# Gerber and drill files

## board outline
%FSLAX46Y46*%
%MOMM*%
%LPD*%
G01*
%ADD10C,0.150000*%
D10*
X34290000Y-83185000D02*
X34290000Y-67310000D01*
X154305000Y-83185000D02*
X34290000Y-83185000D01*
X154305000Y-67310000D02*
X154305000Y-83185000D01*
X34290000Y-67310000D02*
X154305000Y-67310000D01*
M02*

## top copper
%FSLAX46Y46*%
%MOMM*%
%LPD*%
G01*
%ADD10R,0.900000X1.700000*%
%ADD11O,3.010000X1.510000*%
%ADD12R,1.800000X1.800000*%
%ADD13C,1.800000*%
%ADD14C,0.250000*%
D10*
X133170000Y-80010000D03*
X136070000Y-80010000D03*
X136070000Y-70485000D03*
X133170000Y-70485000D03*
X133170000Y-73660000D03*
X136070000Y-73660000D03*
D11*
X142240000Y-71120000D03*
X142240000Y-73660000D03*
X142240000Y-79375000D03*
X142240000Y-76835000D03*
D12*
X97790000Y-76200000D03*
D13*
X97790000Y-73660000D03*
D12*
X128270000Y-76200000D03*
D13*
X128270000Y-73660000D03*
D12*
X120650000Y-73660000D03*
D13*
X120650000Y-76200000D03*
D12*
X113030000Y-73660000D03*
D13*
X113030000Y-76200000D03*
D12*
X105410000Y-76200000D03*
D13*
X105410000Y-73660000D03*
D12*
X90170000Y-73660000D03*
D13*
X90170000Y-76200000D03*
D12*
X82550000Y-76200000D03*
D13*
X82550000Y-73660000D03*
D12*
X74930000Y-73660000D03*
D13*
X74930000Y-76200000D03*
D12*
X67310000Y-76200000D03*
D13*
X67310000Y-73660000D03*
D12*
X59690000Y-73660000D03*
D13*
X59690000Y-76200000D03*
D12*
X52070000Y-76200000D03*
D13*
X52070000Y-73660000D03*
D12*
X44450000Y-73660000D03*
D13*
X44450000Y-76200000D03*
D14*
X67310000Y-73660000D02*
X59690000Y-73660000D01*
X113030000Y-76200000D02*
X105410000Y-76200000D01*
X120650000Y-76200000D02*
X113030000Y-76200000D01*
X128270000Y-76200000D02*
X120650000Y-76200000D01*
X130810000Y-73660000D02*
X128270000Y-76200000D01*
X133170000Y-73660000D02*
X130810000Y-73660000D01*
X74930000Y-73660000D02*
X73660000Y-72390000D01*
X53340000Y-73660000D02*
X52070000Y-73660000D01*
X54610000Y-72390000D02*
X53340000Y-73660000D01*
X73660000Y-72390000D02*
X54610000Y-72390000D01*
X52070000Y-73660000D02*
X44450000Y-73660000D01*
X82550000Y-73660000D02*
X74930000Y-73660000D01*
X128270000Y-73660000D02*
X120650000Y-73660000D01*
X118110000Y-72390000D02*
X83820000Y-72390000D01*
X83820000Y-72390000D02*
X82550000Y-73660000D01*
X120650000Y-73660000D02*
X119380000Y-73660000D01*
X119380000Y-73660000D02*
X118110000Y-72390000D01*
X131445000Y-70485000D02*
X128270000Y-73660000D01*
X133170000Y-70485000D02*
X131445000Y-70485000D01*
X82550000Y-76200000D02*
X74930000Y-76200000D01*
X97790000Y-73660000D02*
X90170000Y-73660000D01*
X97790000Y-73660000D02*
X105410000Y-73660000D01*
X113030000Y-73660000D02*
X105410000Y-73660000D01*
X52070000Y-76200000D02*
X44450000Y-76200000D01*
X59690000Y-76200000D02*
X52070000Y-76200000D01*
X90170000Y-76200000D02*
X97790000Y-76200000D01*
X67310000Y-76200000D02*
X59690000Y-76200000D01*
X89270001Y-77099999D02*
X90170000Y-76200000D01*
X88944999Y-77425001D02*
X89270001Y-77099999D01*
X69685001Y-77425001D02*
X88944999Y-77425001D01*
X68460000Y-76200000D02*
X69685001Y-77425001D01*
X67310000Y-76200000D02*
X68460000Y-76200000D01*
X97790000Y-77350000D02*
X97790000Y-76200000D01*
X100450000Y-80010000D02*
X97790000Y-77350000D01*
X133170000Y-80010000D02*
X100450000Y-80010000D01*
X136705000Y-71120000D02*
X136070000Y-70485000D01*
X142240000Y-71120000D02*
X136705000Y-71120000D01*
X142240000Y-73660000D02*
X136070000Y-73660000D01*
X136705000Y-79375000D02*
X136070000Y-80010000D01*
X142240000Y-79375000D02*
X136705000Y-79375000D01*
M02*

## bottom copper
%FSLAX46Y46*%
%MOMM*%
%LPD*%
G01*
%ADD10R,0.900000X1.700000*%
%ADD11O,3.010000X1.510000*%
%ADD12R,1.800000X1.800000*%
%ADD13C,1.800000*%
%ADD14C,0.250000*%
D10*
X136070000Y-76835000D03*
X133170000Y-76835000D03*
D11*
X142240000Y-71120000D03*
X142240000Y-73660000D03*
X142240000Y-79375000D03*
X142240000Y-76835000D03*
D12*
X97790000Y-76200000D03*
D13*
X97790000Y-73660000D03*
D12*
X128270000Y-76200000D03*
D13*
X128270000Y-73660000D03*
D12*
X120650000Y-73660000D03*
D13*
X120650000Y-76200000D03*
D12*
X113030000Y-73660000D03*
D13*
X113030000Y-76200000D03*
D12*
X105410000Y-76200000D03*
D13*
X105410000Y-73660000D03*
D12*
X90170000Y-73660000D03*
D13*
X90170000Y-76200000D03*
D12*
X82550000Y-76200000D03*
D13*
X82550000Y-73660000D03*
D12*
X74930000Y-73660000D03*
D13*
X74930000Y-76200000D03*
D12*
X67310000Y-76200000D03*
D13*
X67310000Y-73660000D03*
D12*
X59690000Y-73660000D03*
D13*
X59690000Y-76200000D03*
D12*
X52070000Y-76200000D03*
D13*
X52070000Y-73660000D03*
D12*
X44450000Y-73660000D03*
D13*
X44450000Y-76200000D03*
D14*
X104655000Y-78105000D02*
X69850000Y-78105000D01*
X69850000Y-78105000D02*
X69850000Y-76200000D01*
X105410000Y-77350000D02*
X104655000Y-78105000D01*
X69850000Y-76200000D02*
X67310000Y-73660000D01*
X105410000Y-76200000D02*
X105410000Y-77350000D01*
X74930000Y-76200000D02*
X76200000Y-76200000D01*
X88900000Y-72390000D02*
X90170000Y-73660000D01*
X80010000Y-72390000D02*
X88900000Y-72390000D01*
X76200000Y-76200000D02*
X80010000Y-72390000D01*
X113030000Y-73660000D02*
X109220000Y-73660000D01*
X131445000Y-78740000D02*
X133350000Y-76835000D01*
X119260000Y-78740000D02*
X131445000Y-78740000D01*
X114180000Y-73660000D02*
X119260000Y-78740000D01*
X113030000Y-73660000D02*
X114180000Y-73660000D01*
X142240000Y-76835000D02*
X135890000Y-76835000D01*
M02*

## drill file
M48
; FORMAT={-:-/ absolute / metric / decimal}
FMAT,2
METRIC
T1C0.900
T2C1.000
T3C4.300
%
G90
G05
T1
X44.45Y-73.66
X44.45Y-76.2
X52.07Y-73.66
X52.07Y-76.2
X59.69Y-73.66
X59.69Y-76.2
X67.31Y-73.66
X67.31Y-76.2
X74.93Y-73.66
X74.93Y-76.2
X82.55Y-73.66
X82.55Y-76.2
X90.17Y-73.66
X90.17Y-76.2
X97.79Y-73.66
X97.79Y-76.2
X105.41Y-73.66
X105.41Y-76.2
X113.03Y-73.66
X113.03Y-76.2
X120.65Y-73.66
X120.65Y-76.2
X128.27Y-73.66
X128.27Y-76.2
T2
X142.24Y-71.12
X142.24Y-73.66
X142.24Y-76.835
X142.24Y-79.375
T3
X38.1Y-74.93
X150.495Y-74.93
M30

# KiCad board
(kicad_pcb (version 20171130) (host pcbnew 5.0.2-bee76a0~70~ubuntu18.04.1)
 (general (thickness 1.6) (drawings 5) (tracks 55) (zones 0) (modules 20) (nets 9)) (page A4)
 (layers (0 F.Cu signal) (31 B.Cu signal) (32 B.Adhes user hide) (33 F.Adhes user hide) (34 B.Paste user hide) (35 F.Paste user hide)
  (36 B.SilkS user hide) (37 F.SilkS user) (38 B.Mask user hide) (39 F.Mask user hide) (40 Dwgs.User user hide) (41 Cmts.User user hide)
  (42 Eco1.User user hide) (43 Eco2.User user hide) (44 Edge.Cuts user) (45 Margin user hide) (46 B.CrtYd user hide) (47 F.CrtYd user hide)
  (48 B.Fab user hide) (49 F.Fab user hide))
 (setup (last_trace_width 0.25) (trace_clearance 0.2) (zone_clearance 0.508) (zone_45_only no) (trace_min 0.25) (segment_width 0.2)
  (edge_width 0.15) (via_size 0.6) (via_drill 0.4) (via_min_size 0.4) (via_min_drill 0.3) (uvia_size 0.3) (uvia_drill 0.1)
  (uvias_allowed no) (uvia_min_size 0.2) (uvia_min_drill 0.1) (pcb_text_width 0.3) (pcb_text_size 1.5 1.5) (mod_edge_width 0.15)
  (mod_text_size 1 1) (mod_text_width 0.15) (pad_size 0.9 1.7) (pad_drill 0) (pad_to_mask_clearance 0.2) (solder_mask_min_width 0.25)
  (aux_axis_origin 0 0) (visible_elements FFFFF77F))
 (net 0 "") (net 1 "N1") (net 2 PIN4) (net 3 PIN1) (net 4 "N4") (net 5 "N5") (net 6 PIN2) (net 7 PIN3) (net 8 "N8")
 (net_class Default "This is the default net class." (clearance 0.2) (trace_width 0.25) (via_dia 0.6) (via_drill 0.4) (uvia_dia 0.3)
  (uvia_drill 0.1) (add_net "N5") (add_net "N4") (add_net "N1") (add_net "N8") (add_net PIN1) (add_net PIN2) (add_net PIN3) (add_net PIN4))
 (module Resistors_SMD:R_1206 (layer F.Cu) (at 134.62 80.01)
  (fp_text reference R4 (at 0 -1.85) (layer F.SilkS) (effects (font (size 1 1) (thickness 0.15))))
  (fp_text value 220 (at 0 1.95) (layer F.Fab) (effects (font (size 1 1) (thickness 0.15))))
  (pad 1 smd rect (at -1.45 0) (size 0.9 1.7) (layers F.Cu F.Paste F.Mask) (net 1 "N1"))
  (pad 2 smd rect (at 1.45 0) (size 0.9 1.7) (layers F.Cu F.Paste F.Mask) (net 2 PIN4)))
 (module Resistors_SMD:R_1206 (layer F.Cu) (at 134.62 70.485)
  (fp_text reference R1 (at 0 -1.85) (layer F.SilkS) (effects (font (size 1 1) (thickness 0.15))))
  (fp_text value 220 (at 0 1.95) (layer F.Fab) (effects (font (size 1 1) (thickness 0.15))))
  (pad 2 smd rect (at 1.45 0) (size 0.9 1.7) (layers F.Cu F.Paste F.Mask) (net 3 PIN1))
  (pad 1 smd rect (at -1.45 0) (size 0.9 1.7) (layers F.Cu F.Paste F.Mask) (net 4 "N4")))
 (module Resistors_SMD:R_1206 (layer F.Cu) (at 134.62 73.66)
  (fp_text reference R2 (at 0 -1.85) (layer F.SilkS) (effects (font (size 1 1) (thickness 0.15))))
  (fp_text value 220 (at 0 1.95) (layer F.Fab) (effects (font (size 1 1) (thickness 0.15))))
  (pad 1 smd rect (at -1.45 0) (size 0.9 1.7) (layers F.Cu F.Paste F.Mask) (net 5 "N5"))
  (pad 2 smd rect (at 1.45 0) (size 0.9 1.7) (layers F.Cu F.Paste F.Mask) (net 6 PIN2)))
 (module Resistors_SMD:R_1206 (layer F.Cu) (at 134.62 76.835)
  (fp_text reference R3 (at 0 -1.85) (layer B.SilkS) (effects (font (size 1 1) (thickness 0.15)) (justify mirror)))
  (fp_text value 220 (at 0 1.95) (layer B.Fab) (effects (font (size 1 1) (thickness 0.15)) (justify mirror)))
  (pad 2 smd rect (at 1.45 0) (size 0.9 1.7) (layers B.Cu B.Paste B.Mask) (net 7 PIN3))
  (pad 1 smd rect (at -1.45 0) (size 0.9 1.7) (layers B.Cu B.Paste B.Mask) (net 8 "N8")))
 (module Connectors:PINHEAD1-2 (layer F.Cu) (at 142.24 71.12 270)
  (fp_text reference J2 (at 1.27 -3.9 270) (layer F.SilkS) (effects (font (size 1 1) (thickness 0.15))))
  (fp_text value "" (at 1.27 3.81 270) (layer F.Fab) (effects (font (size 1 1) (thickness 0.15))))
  (pad 1 thru_hole oval (at 0 0 270) (size 1.51 3.01) (drill 1) (layers *.Cu *.Mask) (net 3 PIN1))
  (pad 2 thru_hole oval (at 2.54 0 270) (size 1.51 3.01) (drill 1) (layers *.Cu *.Mask) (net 6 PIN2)))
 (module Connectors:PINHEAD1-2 (layer F.Cu) (at 142.24 76.835 270)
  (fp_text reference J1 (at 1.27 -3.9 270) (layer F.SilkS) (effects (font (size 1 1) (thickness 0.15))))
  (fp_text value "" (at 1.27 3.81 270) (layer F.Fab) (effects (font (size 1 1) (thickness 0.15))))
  (pad 2 thru_hole oval (at 2.54 0 270) (size 1.51 3.01) (drill 1) (layers *.Cu *.Mask) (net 2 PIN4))
  (pad 1 thru_hole oval (at 0 0 270) (size 1.51 3.01) (drill 1) (layers *.Cu *.Mask) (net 7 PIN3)))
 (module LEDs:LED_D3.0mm (layer F.Cu) (at 97.79 76.2 90)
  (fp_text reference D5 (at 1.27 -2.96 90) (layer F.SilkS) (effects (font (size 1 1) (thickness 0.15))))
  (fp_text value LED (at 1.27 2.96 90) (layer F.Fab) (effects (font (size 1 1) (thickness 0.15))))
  (pad 1 thru_hole rect (at 0 0 90) (size 1.8 1.8) (drill 0.9) (layers *.Cu *.Mask) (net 1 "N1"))
  (pad 2 thru_hole circle (at 2.54 0 90) (size 1.8 1.8) (drill 0.9) (layers *.Cu *.Mask) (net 8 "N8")))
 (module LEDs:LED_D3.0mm (layer F.Cu) (at 128.27 76.2 90)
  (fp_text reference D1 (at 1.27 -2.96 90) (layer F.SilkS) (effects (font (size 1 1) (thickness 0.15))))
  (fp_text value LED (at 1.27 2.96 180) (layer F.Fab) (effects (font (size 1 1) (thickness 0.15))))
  (pad 1 thru_hole rect (at 0 0 90) (size 1.8 1.8) (drill 0.9) (layers *.Cu *.Mask) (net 5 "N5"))
  (pad 2 thru_hole circle (at 2.54 0 90) (size 1.8 1.8) (drill 0.9) (layers *.Cu *.Mask) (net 4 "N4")))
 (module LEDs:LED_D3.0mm (layer F.Cu) (at 120.65 73.66 270)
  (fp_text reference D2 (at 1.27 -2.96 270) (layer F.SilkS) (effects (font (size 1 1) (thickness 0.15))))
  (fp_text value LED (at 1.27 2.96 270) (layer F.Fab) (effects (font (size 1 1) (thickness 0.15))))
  (pad 1 thru_hole rect (at 0 0 270) (size 1.8 1.8) (drill 0.9) (layers *.Cu *.Mask) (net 4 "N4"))
  (pad 2 thru_hole circle (at 2.54 0 270) (size 1.8 1.8) (drill 0.9) (layers *.Cu *.Mask) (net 5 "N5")))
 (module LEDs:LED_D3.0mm (layer F.Cu) (at 113.03 73.66 270)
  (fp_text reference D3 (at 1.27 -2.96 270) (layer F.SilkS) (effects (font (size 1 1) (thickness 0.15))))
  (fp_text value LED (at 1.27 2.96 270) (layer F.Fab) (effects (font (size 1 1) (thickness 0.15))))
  (pad 1 thru_hole rect (at 0 0 270) (size 1.8 1.8) (drill 0.9) (layers *.Cu *.Mask) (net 8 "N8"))
  (pad 2 thru_hole circle (at 2.54 0 270) (size 1.8 1.8) (drill 0.9) (layers *.Cu *.Mask) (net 5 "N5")))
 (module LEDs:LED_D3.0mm (layer F.Cu) (at 105.41 76.2 90)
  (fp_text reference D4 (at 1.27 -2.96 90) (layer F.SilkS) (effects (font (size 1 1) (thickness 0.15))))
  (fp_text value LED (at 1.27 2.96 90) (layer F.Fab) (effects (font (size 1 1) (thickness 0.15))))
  (pad 1 thru_hole rect (at 0 0 90) (size 1.8 1.8) (drill 0.9) (layers *.Cu *.Mask) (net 5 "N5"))
  (pad 2 thru_hole circle (at 2.54 0 90) (size 1.8 1.8) (drill 0.9) (layers *.Cu *.Mask) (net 8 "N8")))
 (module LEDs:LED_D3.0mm (layer F.Cu) (at 90.17 73.66 270)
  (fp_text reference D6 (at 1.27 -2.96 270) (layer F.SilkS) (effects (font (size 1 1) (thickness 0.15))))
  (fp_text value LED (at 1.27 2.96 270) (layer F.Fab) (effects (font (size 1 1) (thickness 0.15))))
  (pad 1 thru_hole rect (at 0 0 270) (size 1.8 1.8) (drill 0.9) (layers *.Cu *.Mask) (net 8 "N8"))
  (pad 2 thru_hole circle (at 2.54 0 270) (size 1.8 1.8) (drill 0.9) (layers *.Cu *.Mask) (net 1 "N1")))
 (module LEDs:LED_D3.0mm (layer F.Cu) (at 82.55 76.2 90)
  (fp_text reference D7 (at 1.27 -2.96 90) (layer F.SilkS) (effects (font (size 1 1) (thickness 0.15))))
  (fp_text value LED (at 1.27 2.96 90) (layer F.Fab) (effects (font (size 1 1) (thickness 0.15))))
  (pad 1 thru_hole rect (at 0 0 90) (size 1.8 1.8) (drill 0.9) (layers *.Cu *.Mask) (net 8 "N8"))
  (pad 2 thru_hole circle (at 2.54 0 90) (size 1.8 1.8) (drill 0.9) (layers *.Cu *.Mask) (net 4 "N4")))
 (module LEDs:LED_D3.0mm (layer F.Cu) (at 74.93 73.66 270)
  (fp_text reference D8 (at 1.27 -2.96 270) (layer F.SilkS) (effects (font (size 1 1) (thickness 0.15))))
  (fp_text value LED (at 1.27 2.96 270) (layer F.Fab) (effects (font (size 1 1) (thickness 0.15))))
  (pad 1 thru_hole rect (at 0 0 270) (size 1.8 1.8) (drill 0.9) (layers *.Cu *.Mask) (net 4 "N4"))
  (pad 2 thru_hole circle (at 2.54 0 270) (size 1.8 1.8) (drill 0.9) (layers *.Cu *.Mask) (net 8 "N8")))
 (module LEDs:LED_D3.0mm (layer F.Cu) (at 67.31 76.2 90)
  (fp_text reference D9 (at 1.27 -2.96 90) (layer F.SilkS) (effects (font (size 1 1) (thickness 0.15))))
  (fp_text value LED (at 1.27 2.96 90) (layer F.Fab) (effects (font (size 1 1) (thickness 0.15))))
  (pad 1 thru_hole rect (at 0 0 90) (size 1.8 1.8) (drill 0.9) (layers *.Cu *.Mask) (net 1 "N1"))
  (pad 2 thru_hole circle (at 2.54 0 90) (size 1.8 1.8) (drill 0.9) (layers *.Cu *.Mask) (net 5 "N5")))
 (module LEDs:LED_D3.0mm (layer F.Cu) (at 59.69 73.66 270)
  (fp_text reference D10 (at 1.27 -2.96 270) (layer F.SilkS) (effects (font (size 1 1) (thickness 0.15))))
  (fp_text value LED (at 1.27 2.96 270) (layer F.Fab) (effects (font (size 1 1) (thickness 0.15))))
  (pad 1 thru_hole rect (at 0 0 270) (size 1.8 1.8) (drill 0.9) (layers *.Cu *.Mask) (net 5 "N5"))
  (pad 2 thru_hole circle (at 2.54 0 270) (size 1.8 1.8) (drill 0.9) (layers *.Cu *.Mask) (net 1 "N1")))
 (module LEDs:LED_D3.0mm (layer F.Cu) (at 52.07 76.2 90)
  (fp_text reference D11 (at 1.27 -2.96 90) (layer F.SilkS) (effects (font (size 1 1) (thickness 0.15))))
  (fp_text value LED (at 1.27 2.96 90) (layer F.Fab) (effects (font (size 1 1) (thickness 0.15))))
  (pad 1 thru_hole rect (at 0 0 90) (size 1.8 1.8) (drill 0.9) (layers *.Cu *.Mask) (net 1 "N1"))
  (pad 2 thru_hole circle (at 2.54 0 90) (size 1.8 1.8) (drill 0.9) (layers *.Cu *.Mask) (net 4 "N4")))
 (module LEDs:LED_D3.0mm (layer F.Cu) (at 44.45 73.66 270)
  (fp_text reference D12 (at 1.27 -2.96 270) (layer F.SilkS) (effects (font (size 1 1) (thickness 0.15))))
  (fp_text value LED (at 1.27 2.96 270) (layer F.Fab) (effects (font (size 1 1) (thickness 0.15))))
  (pad 1 thru_hole rect (at 0 0 270) (size 1.8 1.8) (drill 0.9) (layers *.Cu *.Mask) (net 4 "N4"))
  (pad 2 thru_hole circle (at 2.54 0 270) (size 1.8 1.8) (drill 0.9) (layers *.Cu *.Mask) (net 1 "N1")))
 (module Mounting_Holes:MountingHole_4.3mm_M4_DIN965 (layer F.Cu) (at 38.1 74.93)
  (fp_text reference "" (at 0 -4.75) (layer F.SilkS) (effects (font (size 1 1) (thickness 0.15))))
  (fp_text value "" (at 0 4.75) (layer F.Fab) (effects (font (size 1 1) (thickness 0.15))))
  (pad 1 np_thru_hole circle (at 0 0) (size 4.3 4.3) (drill 4.3) (layers *.Cu *.Mask)))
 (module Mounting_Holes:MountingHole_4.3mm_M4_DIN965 (layer F.Cu) (at 150.495 74.93)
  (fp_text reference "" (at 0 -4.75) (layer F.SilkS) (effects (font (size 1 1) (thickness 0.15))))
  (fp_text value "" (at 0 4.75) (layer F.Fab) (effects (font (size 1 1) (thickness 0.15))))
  (pad 1 np_thru_hole circle (at 0 0) (size 4.3 4.3) (drill 4.3) (layers *.Cu *.Mask)))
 (gr_line (start 34.29 83.185) (end 34.29 67.31) (layer Edge.Cuts) (width 0.15))
 (gr_line (start 154.305 83.185) (end 34.29 83.185) (layer Edge.Cuts) (width 0.15))
 (gr_line (start 154.305 67.31) (end 154.305 83.185) (layer Edge.Cuts) (width 0.15))
 (gr_line (start 34.29 67.31) (end 154.305 67.31) (layer Edge.Cuts) (width 0.15))
 (segment (start 67.31 73.66) (end 59.69 73.66) (width 0.25) (layer F.Cu) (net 5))
 (segment (start 113.03 76.2) (end 105.41 76.2) (width 0.25) (layer F.Cu) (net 5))
 (segment (start 120.65 76.2) (end 113.03 76.2) (width 0.25) (layer F.Cu) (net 5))
 (segment (start 128.27 76.2) (end 120.65 76.2) (width 0.25) (layer F.Cu) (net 5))
 (segment (start 104.655 78.105) (end 69.85 78.105) (width 0.25) (layer B.Cu) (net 5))
 (segment (start 69.85 78.105) (end 69.85 76.2) (width 0.25) (layer B.Cu) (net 5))
 (segment (start 105.41 77.35) (end 104.655 78.105) (width 0.25) (layer B.Cu) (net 5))
 (segment (start 69.85 76.2) (end 67.31 73.66) (width 0.25) (layer B.Cu) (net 5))
 (segment (start 105.41 76.2) (end 105.41 77.35) (width 0.25) (layer B.Cu) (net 5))
 (segment (start 130.81 73.66) (end 128.27 76.2) (width 0.25) (layer F.Cu) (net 5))
 (segment (start 133.17 73.66) (end 130.81 73.66) (width 0.25) (layer F.Cu) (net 5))
 (segment (start 74.93 73.66) (end 73.66 72.39) (width 0.25) (layer F.Cu) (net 4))
 (segment (start 53.34 73.66) (end 52.07 73.66) (width 0.25) (layer F.Cu) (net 4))
 (segment (start 54.61 72.39) (end 53.34 73.66) (width 0.25) (layer F.Cu) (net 4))
 (segment (start 73.66 72.39) (end 54.61 72.39) (width 0.25) (layer F.Cu) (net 4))
 (segment (start 52.07 73.66) (end 44.45 73.66) (width 0.25) (layer F.Cu) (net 4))
 (segment (start 82.55 73.66) (end 74.93 73.66) (width 0.25) (layer F.Cu) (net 4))
 (segment (start 128.27 73.66) (end 120.65 73.66) (width 0.25) (layer F.Cu) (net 4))
 (segment (start 118.11 72.39) (end 83.82 72.39) (width 0.25) (layer F.Cu) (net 4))
 (segment (start 83.82 72.39) (end 82.55 73.66) (width 0.25) (layer F.Cu) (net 4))
 (segment (start 120.65 73.66) (end 119.38 73.66) (width 0.25) (layer F.Cu) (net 4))
 (segment (start 119.38 73.66) (end 118.11 72.39) (width 0.25) (layer F.Cu) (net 4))
 (segment (start 131.445 70.485) (end 128.27 73.66) (width 0.25) (layer F.Cu) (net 4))
 (segment (start 133.17 70.485) (end 131.445 70.485) (width 0.25) (layer F.Cu) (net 4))
 (segment (start 74.93 76.2) (end 76.2 76.2) (width 0.25) (layer B.Cu) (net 8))
 (segment (start 88.9 72.39) (end 90.17 73.66) (width 0.25) (layer B.Cu) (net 8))
 (segment (start 80.01 72.39) (end 88.9 72.39) (width 0.25) (layer B.Cu) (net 8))
 (segment (start 76.2 76.2) (end 80.01 72.39) (width 0.25) (layer B.Cu) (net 8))
 (segment (start 82.55 76.2) (end 74.93 76.2) (width 0.25) (layer F.Cu) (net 8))
 (segment (start 97.79 73.66) (end 90.17 73.66) (width 0.25) (layer F.Cu) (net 8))
 (segment (start 97.79 73.66) (end 105.41 73.66) (width 0.25) (layer F.Cu) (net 8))
 (segment (start 113.03 73.66) (end 105.41 73.66) (width 0.25) (layer F.Cu) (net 8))
 (segment (start 113.03 73.66) (end 109.22 73.66) (width 0.25) (layer B.Cu) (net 8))
 (segment (start 131.445 78.74) (end 133.35 76.835) (width 0.25) (layer B.Cu) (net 8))
 (segment (start 119.26 78.74) (end 131.445 78.74) (width 0.25) (layer B.Cu) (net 8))
 (segment (start 114.18 73.66) (end 119.26 78.74) (width 0.25) (layer B.Cu) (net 8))
 (segment (start 113.03 73.66) (end 114.18 73.66) (width 0.25) (layer B.Cu) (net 8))
 (segment (start 52.07 76.2) (end 44.45 76.2) (width 0.25) (layer F.Cu) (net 1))
 (segment (start 59.69 76.2) (end 52.07 76.2) (width 0.25) (layer F.Cu) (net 1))
 (segment (start 90.17 76.2) (end 97.79 76.2) (width 0.25) (layer F.Cu) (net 1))
 (segment (start 67.31 76.2) (end 59.69 76.2) (width 0.25) (layer F.Cu) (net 1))
 (segment (start 89.270001 77.099999) (end 90.17 76.2) (width 0.25) (layer F.Cu) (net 1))
 (segment (start 88.944999 77.425001) (end 89.270001 77.099999) (width 0.25) (layer F.Cu) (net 1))
 (segment (start 69.685001 77.425001) (end 88.944999 77.425001) (width 0.25) (layer F.Cu) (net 1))
 (segment (start 68.46 76.2) (end 69.685001 77.425001) (width 0.25) (layer F.Cu) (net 1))
 (segment (start 67.31 76.2) (end 68.46 76.2) (width 0.25) (layer F.Cu) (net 1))
 (segment (start 97.79 77.35) (end 97.79 76.2) (width 0.25) (layer F.Cu) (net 1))
 (segment (start 100.45 80.01) (end 97.79 77.35) (width 0.25) (layer F.Cu) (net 1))
 (segment (start 133.17 80.01) (end 100.45 80.01) (width 0.25) (layer F.Cu) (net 1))
 (segment (start 136.705 71.12) (end 136.07 70.485) (width 0.25) (layer F.Cu) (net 3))
 (segment (start 142.24 71.12) (end 136.705 71.12) (width 0.25) (layer F.Cu) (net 3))
 (segment (start 142.24 73.66) (end 136.07 73.66) (width 0.25) (layer F.Cu) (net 6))
 (segment (start 142.24 76.835) (end 135.89 76.835) (width 0.25) (layer B.Cu) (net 7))
 (segment (start 136.705 79.375) (end 136.07 80.01) (width 0.25) (layer F.Cu) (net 2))
 (segment (start 142.24 79.375) (end 136.705 79.375) (width 0.25) (layer F.Cu) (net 2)))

